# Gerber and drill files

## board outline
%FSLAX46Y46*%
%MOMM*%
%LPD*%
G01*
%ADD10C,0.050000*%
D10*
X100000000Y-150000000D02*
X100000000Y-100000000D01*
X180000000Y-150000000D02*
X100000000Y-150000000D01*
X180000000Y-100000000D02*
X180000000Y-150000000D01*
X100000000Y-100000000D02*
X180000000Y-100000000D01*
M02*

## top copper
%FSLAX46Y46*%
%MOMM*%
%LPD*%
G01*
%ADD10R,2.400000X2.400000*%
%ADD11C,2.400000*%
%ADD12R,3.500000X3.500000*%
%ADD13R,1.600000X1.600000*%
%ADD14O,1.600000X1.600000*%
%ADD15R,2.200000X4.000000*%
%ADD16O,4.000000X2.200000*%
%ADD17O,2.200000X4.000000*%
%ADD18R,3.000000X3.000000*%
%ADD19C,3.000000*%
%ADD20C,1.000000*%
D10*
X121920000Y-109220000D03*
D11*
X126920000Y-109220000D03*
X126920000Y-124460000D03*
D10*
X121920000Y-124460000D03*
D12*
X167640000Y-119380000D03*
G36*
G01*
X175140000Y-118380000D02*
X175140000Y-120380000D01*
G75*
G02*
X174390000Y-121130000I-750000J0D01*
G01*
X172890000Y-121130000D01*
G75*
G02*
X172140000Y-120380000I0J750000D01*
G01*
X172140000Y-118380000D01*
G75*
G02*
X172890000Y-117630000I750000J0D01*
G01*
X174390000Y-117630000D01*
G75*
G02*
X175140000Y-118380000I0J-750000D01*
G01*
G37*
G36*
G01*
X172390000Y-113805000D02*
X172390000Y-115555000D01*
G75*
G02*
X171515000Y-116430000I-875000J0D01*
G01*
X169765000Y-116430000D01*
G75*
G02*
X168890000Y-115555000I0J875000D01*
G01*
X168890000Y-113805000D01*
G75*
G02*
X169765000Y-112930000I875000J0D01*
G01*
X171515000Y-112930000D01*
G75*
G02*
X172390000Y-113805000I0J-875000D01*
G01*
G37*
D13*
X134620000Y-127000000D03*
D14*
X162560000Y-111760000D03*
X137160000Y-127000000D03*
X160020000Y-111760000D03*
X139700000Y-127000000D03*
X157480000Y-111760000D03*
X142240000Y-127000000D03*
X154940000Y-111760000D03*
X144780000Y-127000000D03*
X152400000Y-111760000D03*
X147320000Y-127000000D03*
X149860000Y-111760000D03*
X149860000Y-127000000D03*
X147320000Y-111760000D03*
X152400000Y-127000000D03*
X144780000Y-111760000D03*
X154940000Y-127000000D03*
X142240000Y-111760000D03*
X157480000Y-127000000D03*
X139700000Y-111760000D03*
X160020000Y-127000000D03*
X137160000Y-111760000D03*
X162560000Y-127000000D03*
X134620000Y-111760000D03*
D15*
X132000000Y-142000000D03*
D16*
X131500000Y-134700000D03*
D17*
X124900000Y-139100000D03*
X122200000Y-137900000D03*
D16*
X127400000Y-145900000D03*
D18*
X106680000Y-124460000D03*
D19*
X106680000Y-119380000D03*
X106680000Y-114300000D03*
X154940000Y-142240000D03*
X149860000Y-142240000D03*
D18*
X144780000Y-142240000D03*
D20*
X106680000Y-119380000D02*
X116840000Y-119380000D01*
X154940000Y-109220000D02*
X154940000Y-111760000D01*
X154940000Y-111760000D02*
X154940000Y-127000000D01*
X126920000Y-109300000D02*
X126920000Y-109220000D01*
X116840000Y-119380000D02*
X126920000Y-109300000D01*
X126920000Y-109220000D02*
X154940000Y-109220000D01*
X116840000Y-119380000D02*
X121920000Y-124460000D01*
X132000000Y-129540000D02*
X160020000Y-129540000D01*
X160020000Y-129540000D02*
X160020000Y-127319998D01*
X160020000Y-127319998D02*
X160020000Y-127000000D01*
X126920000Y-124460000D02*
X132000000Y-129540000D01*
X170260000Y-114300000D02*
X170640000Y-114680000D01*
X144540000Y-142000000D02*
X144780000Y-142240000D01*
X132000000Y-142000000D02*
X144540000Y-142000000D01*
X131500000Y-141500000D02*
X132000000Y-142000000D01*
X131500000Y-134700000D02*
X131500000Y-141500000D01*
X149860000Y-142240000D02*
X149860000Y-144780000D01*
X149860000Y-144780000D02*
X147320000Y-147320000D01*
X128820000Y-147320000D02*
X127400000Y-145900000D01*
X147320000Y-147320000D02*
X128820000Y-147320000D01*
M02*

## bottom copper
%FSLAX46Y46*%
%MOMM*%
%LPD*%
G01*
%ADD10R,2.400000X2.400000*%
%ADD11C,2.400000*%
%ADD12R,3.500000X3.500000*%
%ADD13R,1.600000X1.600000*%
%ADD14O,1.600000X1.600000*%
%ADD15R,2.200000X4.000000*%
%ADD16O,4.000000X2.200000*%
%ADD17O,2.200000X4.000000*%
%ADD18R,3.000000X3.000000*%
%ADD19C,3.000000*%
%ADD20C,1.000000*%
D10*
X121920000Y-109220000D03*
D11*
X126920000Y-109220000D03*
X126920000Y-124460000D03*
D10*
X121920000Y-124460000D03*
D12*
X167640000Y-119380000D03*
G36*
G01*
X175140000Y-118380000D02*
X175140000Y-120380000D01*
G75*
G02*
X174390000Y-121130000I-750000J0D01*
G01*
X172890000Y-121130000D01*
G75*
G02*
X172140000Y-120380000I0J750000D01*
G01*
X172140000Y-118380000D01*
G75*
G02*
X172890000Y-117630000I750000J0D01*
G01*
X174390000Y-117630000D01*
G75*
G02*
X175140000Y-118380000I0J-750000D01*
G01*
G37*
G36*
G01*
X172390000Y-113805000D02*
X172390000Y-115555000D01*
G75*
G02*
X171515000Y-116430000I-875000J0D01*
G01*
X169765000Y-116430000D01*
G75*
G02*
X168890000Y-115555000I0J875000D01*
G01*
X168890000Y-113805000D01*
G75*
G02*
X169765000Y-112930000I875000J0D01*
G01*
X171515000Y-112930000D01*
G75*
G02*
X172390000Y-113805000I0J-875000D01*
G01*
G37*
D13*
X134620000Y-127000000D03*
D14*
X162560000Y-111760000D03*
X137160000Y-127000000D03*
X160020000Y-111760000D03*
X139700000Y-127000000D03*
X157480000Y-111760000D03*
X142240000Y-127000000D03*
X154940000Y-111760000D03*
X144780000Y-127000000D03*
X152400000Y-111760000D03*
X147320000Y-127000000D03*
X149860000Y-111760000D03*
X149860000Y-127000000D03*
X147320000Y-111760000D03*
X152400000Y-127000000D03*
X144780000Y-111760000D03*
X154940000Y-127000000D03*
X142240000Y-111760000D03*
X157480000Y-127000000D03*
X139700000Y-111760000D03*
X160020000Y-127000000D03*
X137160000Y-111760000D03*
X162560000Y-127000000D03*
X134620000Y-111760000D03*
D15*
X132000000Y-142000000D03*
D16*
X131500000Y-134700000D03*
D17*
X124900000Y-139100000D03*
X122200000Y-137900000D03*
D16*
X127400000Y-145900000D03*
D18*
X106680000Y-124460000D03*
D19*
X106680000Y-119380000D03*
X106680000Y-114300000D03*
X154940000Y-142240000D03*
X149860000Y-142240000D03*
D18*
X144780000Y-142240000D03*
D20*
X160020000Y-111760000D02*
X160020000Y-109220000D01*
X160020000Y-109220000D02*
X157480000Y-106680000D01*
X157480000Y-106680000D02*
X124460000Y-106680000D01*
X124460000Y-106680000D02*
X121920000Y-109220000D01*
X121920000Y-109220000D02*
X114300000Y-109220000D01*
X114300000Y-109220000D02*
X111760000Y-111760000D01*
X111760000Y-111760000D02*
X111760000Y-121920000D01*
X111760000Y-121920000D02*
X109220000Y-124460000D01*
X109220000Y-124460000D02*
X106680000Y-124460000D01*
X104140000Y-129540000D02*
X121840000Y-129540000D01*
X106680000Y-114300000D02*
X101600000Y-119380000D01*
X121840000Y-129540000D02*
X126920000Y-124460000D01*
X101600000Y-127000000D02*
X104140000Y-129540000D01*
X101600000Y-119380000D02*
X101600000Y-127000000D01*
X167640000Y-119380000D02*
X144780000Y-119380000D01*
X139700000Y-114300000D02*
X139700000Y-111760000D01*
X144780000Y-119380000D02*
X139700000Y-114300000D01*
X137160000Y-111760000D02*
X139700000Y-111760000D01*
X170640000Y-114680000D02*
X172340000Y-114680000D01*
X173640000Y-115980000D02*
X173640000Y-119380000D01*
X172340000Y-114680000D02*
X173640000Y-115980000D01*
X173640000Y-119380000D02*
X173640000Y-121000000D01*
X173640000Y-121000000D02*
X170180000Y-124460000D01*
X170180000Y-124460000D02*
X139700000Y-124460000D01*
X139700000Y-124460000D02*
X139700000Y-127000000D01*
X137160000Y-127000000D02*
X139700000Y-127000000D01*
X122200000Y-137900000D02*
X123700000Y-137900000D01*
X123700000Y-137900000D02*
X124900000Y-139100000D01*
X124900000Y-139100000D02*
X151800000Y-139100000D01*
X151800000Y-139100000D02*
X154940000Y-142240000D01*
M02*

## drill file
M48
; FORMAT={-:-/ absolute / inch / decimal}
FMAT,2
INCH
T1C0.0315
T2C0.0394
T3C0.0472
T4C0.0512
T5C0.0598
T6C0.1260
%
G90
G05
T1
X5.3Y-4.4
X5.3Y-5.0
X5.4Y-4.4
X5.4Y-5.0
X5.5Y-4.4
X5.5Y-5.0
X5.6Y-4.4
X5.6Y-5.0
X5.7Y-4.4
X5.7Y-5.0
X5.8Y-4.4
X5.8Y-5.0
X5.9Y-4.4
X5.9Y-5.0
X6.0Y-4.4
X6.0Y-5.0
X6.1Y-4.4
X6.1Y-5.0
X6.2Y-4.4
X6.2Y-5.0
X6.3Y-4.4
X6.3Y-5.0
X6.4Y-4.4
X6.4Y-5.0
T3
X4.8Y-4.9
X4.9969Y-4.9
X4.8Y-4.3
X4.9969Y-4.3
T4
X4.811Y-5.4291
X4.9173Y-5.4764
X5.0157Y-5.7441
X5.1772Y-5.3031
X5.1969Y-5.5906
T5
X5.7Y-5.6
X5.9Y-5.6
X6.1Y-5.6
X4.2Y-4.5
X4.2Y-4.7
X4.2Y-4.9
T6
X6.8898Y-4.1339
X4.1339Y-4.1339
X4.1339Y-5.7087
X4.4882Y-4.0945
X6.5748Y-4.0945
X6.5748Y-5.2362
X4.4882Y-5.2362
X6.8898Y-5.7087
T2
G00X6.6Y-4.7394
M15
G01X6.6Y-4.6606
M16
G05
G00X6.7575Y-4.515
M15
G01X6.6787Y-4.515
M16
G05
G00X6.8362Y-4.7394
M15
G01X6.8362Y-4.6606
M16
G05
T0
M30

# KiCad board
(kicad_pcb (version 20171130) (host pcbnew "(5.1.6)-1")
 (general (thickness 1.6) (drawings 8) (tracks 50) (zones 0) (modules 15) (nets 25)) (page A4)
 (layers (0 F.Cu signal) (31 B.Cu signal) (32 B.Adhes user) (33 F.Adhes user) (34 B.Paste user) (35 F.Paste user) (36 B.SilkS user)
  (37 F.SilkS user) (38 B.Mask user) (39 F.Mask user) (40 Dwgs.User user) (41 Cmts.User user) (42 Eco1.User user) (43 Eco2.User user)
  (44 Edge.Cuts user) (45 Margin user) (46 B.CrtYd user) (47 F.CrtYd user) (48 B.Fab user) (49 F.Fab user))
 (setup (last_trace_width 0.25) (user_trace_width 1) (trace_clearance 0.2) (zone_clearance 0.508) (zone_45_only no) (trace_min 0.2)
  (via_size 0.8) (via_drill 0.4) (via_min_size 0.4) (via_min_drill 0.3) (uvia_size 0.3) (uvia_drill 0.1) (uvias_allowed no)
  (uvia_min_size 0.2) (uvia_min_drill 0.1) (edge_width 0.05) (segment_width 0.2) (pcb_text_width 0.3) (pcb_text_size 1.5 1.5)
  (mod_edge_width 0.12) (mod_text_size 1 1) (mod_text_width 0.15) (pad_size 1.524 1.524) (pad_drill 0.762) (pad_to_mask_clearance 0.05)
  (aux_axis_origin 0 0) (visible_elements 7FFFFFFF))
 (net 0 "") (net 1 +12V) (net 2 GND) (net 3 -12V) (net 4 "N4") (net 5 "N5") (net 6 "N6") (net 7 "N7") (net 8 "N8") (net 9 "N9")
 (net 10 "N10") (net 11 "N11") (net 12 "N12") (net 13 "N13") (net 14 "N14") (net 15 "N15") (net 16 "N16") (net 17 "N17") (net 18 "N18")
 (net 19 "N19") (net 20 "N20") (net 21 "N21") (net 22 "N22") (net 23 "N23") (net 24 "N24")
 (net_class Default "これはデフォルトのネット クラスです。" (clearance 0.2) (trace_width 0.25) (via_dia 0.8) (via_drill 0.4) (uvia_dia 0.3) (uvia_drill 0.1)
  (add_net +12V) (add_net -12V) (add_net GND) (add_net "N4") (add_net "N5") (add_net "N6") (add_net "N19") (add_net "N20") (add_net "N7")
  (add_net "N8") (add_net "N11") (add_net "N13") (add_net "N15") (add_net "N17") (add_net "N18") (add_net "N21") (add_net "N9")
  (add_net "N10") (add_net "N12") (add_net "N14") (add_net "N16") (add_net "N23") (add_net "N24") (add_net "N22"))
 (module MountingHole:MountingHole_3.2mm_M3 (layer F.Cu) (at 167 133)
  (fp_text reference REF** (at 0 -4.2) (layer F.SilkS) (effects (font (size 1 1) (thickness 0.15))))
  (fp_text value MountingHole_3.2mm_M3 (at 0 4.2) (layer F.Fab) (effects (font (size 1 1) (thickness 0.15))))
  (pad 1 np_thru_hole circle (at 0 0) (size 3.2 3.2) (drill 3.2) (layers *.Cu *.Mask)))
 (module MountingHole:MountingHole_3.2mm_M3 (layer F.Cu) (at 167 104)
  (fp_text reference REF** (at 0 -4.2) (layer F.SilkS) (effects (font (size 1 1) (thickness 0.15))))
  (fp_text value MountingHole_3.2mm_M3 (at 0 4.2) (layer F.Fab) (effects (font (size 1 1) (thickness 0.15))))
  (pad 1 np_thru_hole circle (at 0 0) (size 3.2 3.2) (drill 3.2) (layers *.Cu *.Mask)))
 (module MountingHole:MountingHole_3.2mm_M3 (layer F.Cu) (at 114 133)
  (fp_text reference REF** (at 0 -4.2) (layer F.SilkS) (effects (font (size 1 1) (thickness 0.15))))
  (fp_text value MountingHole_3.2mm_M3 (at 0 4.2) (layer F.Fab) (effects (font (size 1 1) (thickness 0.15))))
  (pad 1 np_thru_hole circle (at 0 0) (size 3.2 3.2) (drill 3.2) (layers *.Cu *.Mask)))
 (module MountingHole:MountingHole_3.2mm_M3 (layer F.Cu) (at 114 104)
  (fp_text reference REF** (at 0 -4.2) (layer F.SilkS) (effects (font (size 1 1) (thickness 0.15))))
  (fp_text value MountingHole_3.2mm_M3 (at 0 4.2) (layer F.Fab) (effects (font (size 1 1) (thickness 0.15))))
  (pad 1 np_thru_hole circle (at 0 0) (size 3.2 3.2) (drill 3.2) (layers *.Cu *.Mask)))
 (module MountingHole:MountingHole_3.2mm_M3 (layer F.Cu) (at 175 145)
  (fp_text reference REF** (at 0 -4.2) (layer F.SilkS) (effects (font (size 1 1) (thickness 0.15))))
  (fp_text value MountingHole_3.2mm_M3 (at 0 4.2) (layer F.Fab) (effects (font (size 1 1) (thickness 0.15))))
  (pad 1 np_thru_hole circle (at 0 0) (size 3.2 3.2) (drill 3.2) (layers *.Cu *.Mask)))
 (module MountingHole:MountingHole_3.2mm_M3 (layer F.Cu) (at 105 145)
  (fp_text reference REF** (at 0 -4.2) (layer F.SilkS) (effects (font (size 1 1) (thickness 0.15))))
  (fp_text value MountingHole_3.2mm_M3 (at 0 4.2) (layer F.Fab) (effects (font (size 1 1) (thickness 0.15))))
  (pad 1 np_thru_hole circle (at 0 0) (size 3.2 3.2) (drill 3.2) (layers *.Cu *.Mask)))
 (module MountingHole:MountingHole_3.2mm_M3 (layer F.Cu) (at 175 105)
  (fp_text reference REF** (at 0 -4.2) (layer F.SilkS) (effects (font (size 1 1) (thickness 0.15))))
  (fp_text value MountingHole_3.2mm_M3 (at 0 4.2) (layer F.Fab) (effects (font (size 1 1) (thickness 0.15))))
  (pad 1 np_thru_hole circle (at 0 0) (size 3.2 3.2) (drill 3.2) (layers *.Cu *.Mask)))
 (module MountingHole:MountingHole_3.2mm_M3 (layer F.Cu) (at 105 105)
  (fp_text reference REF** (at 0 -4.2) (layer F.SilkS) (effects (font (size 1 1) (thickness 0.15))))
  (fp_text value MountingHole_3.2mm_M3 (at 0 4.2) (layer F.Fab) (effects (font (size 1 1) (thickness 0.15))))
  (pad 1 np_thru_hole circle (at 0 0) (size 3.2 3.2) (drill 3.2) (layers *.Cu *.Mask)))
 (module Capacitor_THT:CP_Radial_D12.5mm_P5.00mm (layer F.Cu) (at 121.92 109.22)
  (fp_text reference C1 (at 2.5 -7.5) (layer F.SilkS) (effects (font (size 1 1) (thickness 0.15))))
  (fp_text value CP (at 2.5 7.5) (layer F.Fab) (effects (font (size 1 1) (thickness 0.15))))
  (pad 1 thru_hole rect (at 0 0) (size 2.4 2.4) (drill 1.2) (layers *.Cu *.Mask) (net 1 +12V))
  (pad 2 thru_hole circle (at 5 0) (size 2.4 2.4) (drill 1.2) (layers *.Cu *.Mask) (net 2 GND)))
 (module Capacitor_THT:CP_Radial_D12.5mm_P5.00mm (layer F.Cu) (at 121.92 124.46)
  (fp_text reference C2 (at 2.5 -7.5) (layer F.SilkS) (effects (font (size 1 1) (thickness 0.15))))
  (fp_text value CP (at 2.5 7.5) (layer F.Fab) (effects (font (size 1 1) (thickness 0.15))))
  (pad 2 thru_hole circle (at 5 0) (size 2.4 2.4) (drill 1.2) (layers *.Cu *.Mask) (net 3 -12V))
  (pad 1 thru_hole rect (at 0 0) (size 2.4 2.4) (drill 1.2) (layers *.Cu *.Mask) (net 2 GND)))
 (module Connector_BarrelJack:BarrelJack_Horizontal (layer F.Cu) (at 167.64 119.38 180)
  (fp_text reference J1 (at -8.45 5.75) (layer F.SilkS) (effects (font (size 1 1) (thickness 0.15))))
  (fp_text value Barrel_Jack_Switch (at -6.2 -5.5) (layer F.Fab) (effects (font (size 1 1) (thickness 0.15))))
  (pad 1 thru_hole rect (at 0 0 180) (size 3.5 3.5) (drill oval 1 3) (layers *.Cu *.Mask) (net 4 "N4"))
  (pad 2 thru_hole roundrect (at -6 0 180) (size 3 3.5) (drill oval 1 3) (layers *.Cu *.Mask) (roundrect_rratio 0.25) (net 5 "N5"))
  (pad 3 thru_hole roundrect (at -3 4.7 180) (size 3.5 3.5) (drill oval 3 1) (layers *.Cu *.Mask) (roundrect_rratio 0.25) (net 5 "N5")))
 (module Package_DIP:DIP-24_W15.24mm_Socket (layer F.Cu) (at 134.62 127 90)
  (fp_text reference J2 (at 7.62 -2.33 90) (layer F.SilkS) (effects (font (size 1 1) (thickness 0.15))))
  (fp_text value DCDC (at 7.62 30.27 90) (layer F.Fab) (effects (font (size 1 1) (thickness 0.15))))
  (pad 1 thru_hole rect (at 0 0 90) (size 1.6 1.6) (drill 0.8) (layers *.Cu *.Mask) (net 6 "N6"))
  (pad 13 thru_hole oval (at 15.24 27.94 90) (size 1.6 1.6) (drill 0.8) (layers *.Cu *.Mask) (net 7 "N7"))
  (pad 2 thru_hole oval (at 0 2.54 90) (size 1.6 1.6) (drill 0.8) (layers *.Cu *.Mask) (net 5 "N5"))
  (pad 14 thru_hole oval (at 15.24 25.4 90) (size 1.6 1.6) (drill 0.8) (layers *.Cu *.Mask) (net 1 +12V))
  (pad 3 thru_hole oval (at 0 5.08 90) (size 1.6 1.6) (drill 0.8) (layers *.Cu *.Mask) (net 5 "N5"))
  (pad 15 thru_hole oval (at 15.24 22.86 90) (size 1.6 1.6) (drill 0.8) (layers *.Cu *.Mask) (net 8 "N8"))
  (pad 4 thru_hole oval (at 0 7.62 90) (size 1.6 1.6) (drill 0.8) (layers *.Cu *.Mask) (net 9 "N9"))
  (pad 16 thru_hole oval (at 15.24 20.32 90) (size 1.6 1.6) (drill 0.8) (layers *.Cu *.Mask) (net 2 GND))
  (pad 5 thru_hole oval (at 0 10.16 90) (size 1.6 1.6) (drill 0.8) (layers *.Cu *.Mask) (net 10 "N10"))
  (pad 17 thru_hole oval (at 15.24 17.78 90) (size 1.6 1.6) (drill 0.8) (layers *.Cu *.Mask) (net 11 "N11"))
  (pad 6 thru_hole oval (at 0 12.7 90) (size 1.6 1.6) (drill 0.8) (layers *.Cu *.Mask) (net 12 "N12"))
  (pad 18 thru_hole oval (at 15.24 15.24 90) (size 1.6 1.6) (drill 0.8) (layers *.Cu *.Mask) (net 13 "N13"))
  (pad 7 thru_hole oval (at 0 15.24 90) (size 1.6 1.6) (drill 0.8) (layers *.Cu *.Mask) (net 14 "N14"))
  (pad 19 thru_hole oval (at 15.24 12.7 90) (size 1.6 1.6) (drill 0.8) (layers *.Cu *.Mask) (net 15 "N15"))
  (pad 8 thru_hole oval (at 0 17.78 90) (size 1.6 1.6) (drill 0.8) (layers *.Cu *.Mask) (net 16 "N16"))
  (pad 20 thru_hole oval (at 15.24 10.16 90) (size 1.6 1.6) (drill 0.8) (layers *.Cu *.Mask) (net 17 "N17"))
  (pad 9 thru_hole oval (at 0 20.32 90) (size 1.6 1.6) (drill 0.8) (layers *.Cu *.Mask) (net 2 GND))
  (pad 21 thru_hole oval (at 15.24 7.62 90) (size 1.6 1.6) (drill 0.8) (layers *.Cu *.Mask) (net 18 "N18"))
  (pad 10 thru_hole oval (at 0 22.86 90) (size 1.6 1.6) (drill 0.8) (layers *.Cu *.Mask) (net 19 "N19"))
  (pad 22 thru_hole oval (at 15.24 5.08 90) (size 1.6 1.6) (drill 0.8) (layers *.Cu *.Mask) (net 4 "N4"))
  (pad 11 thru_hole oval (at 0 25.4 90) (size 1.6 1.6) (drill 0.8) (layers *.Cu *.Mask) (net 3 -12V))
  (pad 23 thru_hole oval (at 15.24 2.54 90) (size 1.6 1.6) (drill 0.8) (layers *.Cu *.Mask) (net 4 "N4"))
  (pad 12 thru_hole oval (at 0 27.94 90) (size 1.6 1.6) (drill 0.8) (layers *.Cu *.Mask) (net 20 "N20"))
  (pad 24 thru_hole oval (at 15.24 0 90) (size 1.6 1.6) (drill 0.8) (layers *.Cu *.Mask) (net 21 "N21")))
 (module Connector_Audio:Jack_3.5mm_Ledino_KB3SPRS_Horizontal (layer F.Cu) (at 132 142 90)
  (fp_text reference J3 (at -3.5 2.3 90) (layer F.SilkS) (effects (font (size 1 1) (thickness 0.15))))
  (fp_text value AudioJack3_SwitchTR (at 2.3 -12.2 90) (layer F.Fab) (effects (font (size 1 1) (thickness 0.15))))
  (pad T thru_hole rect (at 0 0 90) (size 4 2.2) (drill 1.3) (layers *.Cu *.Mask) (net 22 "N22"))
  (pad TN thru_hole oval (at 7.3 -0.5 180) (size 4 2.2) (drill 1.3) (layers *.Cu *.Mask) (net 22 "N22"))
  (pad RN thru_hole oval (at 2.9 -7.1 90) (size 4 2.2) (drill 1.3) (layers *.Cu *.Mask) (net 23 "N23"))
  (pad R thru_hole oval (at 4.1 -9.8 90) (size 4 2.2) (drill 1.3) (layers *.Cu *.Mask) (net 23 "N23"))
  (pad S thru_hole oval (at -3.9 -4.6 90) (size 2.2 4) (drill 1.3) (layers *.Cu *.Mask) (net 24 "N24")))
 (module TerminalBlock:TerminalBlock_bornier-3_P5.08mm (layer F.Cu) (at 106.68 124.46 90)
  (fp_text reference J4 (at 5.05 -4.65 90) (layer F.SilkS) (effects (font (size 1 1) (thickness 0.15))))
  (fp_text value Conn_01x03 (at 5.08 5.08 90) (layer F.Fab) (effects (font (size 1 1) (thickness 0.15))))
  (pad 1 thru_hole rect (at 0 0 90) (size 3 3) (drill 1.52) (layers *.Cu *.Mask) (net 1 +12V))
  (pad 2 thru_hole circle (at 5.08 0 90) (size 3 3) (drill 1.52) (layers *.Cu *.Mask) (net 2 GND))
  (pad 3 thru_hole circle (at 10.16 0 90) (size 3 3) (drill 1.52) (layers *.Cu *.Mask) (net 3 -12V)))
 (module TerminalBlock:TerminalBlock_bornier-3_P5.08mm (layer F.Cu) (at 144.78 142.24)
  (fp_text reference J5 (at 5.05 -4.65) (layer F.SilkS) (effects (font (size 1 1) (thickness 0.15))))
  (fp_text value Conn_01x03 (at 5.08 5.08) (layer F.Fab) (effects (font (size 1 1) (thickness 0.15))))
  (pad 3 thru_hole circle (at 10.16 0) (size 3 3) (drill 1.52) (layers *.Cu *.Mask) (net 23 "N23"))
  (pad 2 thru_hole circle (at 5.08 0) (size 3 3) (drill 1.52) (layers *.Cu *.Mask) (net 24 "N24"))
  (pad 1 thru_hole rect (at 0 0) (size 3 3) (drill 1.52) (layers *.Cu *.Mask) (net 22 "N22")))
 (gr_line (start 100 150) (end 100 100) (layer Edge.Cuts) (width 0.05))
 (gr_line (start 180 150) (end 100 150) (layer Edge.Cuts) (width 0.05))
 (gr_line (start 180 100) (end 180 150) (layer Edge.Cuts) (width 0.05))
 (gr_line (start 100 100) (end 180 100) (layer Edge.Cuts) (width 0.05))
 (segment (start 160.02 111.76) (end 160.02 109.22) (width 1) (layer B.Cu) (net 1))
 (segment (start 160.02 109.22) (end 157.48 106.68) (width 1) (layer B.Cu) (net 1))
 (segment (start 157.48 106.68) (end 124.46 106.68) (width 1) (layer B.Cu) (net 1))
 (segment (start 124.46 106.68) (end 121.92 109.22) (width 1) (layer B.Cu) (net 1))
 (segment (start 121.92 109.22) (end 114.3 109.22) (width 1) (layer B.Cu) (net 1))
 (segment (start 114.3 109.22) (end 111.76 111.76) (width 1) (layer B.Cu) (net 1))
 (segment (start 111.76 111.76) (end 111.76 121.92) (width 1) (layer B.Cu) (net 1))
 (segment (start 111.76 121.92) (end 109.22 124.46) (width 1) (layer B.Cu) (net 1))
 (segment (start 109.22 124.46) (end 106.68 124.46) (width 1) (layer B.Cu) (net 1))
 (segment (start 106.68 119.38) (end 116.84 119.38) (width 1) (layer F.Cu) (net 2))
 (segment (start 154.94 109.22) (end 154.94 111.76) (width 1) (layer F.Cu) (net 2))
 (segment (start 154.94 111.76) (end 154.94 127) (width 1) (layer F.Cu) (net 2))
 (segment (start 126.92 109.3) (end 126.92 109.22) (width 1) (layer F.Cu) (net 2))
 (segment (start 116.84 119.38) (end 126.92 109.3) (width 1) (layer F.Cu) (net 2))
 (segment (start 126.92 109.22) (end 154.94 109.22) (width 1) (layer F.Cu) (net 2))
 (segment (start 116.84 119.38) (end 121.92 124.46) (width 1) (layer F.Cu) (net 2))
 (segment (start 132 129.54) (end 160.02 129.54) (width 1) (layer F.Cu) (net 3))
 (segment (start 160.02 129.54) (end 160.02 127.319998) (width 1) (layer F.Cu) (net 3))
 (segment (start 160.02 127.319998) (end 160.02 127) (width 1) (layer F.Cu) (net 3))
 (segment (start 126.92 124.46) (end 132 129.54) (width 1) (layer F.Cu) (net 3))
 (segment (start 104.14 129.54) (end 121.84 129.54) (width 1) (layer B.Cu) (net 3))
 (segment (start 106.68 114.3) (end 101.6 119.38) (width 1) (layer B.Cu) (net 3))
 (segment (start 121.84 129.54) (end 126.92 124.46) (width 1) (layer B.Cu) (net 3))
 (segment (start 101.6 127) (end 104.14 129.54) (width 1) (layer B.Cu) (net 3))
 (segment (start 101.6 119.38) (end 101.6 127) (width 1) (layer B.Cu) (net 3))
 (segment (start 167.64 119.38) (end 144.78 119.38) (width 1) (layer B.Cu) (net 4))
 (segment (start 139.7 114.3) (end 139.7 111.76) (width 1) (layer B.Cu) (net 4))
 (segment (start 144.78 119.38) (end 139.7 114.3) (width 1) (layer B.Cu) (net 4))
 (segment (start 137.16 111.76) (end 139.7 111.76) (width 1) (layer B.Cu) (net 4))
 (segment (start 170.26 114.3) (end 170.64 114.68) (width 1) (layer F.Cu) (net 5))
 (segment (start 170.64 114.68) (end 172.34 114.68) (width 1) (layer B.Cu) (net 5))
 (segment (start 173.64 115.98) (end 173.64 119.38) (width 1) (layer B.Cu) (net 5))
 (segment (start 172.34 114.68) (end 173.64 115.98) (width 1) (layer B.Cu) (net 5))
 (segment (start 173.64 119.38) (end 173.64 121) (width 1) (layer B.Cu) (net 5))
 (segment (start 173.64 121) (end 170.18 124.46) (width 1) (layer B.Cu) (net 5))
 (segment (start 170.18 124.46) (end 139.7 124.46) (width 1) (layer B.Cu) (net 5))
 (segment (start 139.7 124.46) (end 139.7 127) (width 1) (layer B.Cu) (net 5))
 (segment (start 137.16 127) (end 139.7 127) (width 1) (layer B.Cu) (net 5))
 (segment (start 144.54 142) (end 144.78 142.24) (width 1) (layer F.Cu) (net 22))
 (segment (start 132 142) (end 144.54 142) (width 1) (layer F.Cu) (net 22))
 (segment (start 131.5 141.5) (end 132 142) (width 1) (layer F.Cu) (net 22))
 (segment (start 131.5 134.7) (end 131.5 141.5) (width 1) (layer F.Cu) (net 22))
 (segment (start 122.2 137.9) (end 123.7 137.9) (width 1) (layer B.Cu) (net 23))
 (segment (start 123.7 137.9) (end 124.9 139.1) (width 1) (layer B.Cu) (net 23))
 (segment (start 124.9 139.1) (end 151.8 139.1) (width 1) (layer B.Cu) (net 23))
 (segment (start 151.8 139.1) (end 154.94 142.24) (width 1) (layer B.Cu) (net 23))
 (segment (start 149.86 142.24) (end 149.86 144.78) (width 1) (layer F.Cu) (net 24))
 (segment (start 149.86 144.78) (end 147.32 147.32) (width 1) (layer F.Cu) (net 24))
 (segment (start 128.82 147.32) (end 127.4 145.9) (width 1) (layer F.Cu) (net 24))
 (segment (start 147.32 147.32) (end 128.82 147.32) (width 1) (layer F.Cu) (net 24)))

